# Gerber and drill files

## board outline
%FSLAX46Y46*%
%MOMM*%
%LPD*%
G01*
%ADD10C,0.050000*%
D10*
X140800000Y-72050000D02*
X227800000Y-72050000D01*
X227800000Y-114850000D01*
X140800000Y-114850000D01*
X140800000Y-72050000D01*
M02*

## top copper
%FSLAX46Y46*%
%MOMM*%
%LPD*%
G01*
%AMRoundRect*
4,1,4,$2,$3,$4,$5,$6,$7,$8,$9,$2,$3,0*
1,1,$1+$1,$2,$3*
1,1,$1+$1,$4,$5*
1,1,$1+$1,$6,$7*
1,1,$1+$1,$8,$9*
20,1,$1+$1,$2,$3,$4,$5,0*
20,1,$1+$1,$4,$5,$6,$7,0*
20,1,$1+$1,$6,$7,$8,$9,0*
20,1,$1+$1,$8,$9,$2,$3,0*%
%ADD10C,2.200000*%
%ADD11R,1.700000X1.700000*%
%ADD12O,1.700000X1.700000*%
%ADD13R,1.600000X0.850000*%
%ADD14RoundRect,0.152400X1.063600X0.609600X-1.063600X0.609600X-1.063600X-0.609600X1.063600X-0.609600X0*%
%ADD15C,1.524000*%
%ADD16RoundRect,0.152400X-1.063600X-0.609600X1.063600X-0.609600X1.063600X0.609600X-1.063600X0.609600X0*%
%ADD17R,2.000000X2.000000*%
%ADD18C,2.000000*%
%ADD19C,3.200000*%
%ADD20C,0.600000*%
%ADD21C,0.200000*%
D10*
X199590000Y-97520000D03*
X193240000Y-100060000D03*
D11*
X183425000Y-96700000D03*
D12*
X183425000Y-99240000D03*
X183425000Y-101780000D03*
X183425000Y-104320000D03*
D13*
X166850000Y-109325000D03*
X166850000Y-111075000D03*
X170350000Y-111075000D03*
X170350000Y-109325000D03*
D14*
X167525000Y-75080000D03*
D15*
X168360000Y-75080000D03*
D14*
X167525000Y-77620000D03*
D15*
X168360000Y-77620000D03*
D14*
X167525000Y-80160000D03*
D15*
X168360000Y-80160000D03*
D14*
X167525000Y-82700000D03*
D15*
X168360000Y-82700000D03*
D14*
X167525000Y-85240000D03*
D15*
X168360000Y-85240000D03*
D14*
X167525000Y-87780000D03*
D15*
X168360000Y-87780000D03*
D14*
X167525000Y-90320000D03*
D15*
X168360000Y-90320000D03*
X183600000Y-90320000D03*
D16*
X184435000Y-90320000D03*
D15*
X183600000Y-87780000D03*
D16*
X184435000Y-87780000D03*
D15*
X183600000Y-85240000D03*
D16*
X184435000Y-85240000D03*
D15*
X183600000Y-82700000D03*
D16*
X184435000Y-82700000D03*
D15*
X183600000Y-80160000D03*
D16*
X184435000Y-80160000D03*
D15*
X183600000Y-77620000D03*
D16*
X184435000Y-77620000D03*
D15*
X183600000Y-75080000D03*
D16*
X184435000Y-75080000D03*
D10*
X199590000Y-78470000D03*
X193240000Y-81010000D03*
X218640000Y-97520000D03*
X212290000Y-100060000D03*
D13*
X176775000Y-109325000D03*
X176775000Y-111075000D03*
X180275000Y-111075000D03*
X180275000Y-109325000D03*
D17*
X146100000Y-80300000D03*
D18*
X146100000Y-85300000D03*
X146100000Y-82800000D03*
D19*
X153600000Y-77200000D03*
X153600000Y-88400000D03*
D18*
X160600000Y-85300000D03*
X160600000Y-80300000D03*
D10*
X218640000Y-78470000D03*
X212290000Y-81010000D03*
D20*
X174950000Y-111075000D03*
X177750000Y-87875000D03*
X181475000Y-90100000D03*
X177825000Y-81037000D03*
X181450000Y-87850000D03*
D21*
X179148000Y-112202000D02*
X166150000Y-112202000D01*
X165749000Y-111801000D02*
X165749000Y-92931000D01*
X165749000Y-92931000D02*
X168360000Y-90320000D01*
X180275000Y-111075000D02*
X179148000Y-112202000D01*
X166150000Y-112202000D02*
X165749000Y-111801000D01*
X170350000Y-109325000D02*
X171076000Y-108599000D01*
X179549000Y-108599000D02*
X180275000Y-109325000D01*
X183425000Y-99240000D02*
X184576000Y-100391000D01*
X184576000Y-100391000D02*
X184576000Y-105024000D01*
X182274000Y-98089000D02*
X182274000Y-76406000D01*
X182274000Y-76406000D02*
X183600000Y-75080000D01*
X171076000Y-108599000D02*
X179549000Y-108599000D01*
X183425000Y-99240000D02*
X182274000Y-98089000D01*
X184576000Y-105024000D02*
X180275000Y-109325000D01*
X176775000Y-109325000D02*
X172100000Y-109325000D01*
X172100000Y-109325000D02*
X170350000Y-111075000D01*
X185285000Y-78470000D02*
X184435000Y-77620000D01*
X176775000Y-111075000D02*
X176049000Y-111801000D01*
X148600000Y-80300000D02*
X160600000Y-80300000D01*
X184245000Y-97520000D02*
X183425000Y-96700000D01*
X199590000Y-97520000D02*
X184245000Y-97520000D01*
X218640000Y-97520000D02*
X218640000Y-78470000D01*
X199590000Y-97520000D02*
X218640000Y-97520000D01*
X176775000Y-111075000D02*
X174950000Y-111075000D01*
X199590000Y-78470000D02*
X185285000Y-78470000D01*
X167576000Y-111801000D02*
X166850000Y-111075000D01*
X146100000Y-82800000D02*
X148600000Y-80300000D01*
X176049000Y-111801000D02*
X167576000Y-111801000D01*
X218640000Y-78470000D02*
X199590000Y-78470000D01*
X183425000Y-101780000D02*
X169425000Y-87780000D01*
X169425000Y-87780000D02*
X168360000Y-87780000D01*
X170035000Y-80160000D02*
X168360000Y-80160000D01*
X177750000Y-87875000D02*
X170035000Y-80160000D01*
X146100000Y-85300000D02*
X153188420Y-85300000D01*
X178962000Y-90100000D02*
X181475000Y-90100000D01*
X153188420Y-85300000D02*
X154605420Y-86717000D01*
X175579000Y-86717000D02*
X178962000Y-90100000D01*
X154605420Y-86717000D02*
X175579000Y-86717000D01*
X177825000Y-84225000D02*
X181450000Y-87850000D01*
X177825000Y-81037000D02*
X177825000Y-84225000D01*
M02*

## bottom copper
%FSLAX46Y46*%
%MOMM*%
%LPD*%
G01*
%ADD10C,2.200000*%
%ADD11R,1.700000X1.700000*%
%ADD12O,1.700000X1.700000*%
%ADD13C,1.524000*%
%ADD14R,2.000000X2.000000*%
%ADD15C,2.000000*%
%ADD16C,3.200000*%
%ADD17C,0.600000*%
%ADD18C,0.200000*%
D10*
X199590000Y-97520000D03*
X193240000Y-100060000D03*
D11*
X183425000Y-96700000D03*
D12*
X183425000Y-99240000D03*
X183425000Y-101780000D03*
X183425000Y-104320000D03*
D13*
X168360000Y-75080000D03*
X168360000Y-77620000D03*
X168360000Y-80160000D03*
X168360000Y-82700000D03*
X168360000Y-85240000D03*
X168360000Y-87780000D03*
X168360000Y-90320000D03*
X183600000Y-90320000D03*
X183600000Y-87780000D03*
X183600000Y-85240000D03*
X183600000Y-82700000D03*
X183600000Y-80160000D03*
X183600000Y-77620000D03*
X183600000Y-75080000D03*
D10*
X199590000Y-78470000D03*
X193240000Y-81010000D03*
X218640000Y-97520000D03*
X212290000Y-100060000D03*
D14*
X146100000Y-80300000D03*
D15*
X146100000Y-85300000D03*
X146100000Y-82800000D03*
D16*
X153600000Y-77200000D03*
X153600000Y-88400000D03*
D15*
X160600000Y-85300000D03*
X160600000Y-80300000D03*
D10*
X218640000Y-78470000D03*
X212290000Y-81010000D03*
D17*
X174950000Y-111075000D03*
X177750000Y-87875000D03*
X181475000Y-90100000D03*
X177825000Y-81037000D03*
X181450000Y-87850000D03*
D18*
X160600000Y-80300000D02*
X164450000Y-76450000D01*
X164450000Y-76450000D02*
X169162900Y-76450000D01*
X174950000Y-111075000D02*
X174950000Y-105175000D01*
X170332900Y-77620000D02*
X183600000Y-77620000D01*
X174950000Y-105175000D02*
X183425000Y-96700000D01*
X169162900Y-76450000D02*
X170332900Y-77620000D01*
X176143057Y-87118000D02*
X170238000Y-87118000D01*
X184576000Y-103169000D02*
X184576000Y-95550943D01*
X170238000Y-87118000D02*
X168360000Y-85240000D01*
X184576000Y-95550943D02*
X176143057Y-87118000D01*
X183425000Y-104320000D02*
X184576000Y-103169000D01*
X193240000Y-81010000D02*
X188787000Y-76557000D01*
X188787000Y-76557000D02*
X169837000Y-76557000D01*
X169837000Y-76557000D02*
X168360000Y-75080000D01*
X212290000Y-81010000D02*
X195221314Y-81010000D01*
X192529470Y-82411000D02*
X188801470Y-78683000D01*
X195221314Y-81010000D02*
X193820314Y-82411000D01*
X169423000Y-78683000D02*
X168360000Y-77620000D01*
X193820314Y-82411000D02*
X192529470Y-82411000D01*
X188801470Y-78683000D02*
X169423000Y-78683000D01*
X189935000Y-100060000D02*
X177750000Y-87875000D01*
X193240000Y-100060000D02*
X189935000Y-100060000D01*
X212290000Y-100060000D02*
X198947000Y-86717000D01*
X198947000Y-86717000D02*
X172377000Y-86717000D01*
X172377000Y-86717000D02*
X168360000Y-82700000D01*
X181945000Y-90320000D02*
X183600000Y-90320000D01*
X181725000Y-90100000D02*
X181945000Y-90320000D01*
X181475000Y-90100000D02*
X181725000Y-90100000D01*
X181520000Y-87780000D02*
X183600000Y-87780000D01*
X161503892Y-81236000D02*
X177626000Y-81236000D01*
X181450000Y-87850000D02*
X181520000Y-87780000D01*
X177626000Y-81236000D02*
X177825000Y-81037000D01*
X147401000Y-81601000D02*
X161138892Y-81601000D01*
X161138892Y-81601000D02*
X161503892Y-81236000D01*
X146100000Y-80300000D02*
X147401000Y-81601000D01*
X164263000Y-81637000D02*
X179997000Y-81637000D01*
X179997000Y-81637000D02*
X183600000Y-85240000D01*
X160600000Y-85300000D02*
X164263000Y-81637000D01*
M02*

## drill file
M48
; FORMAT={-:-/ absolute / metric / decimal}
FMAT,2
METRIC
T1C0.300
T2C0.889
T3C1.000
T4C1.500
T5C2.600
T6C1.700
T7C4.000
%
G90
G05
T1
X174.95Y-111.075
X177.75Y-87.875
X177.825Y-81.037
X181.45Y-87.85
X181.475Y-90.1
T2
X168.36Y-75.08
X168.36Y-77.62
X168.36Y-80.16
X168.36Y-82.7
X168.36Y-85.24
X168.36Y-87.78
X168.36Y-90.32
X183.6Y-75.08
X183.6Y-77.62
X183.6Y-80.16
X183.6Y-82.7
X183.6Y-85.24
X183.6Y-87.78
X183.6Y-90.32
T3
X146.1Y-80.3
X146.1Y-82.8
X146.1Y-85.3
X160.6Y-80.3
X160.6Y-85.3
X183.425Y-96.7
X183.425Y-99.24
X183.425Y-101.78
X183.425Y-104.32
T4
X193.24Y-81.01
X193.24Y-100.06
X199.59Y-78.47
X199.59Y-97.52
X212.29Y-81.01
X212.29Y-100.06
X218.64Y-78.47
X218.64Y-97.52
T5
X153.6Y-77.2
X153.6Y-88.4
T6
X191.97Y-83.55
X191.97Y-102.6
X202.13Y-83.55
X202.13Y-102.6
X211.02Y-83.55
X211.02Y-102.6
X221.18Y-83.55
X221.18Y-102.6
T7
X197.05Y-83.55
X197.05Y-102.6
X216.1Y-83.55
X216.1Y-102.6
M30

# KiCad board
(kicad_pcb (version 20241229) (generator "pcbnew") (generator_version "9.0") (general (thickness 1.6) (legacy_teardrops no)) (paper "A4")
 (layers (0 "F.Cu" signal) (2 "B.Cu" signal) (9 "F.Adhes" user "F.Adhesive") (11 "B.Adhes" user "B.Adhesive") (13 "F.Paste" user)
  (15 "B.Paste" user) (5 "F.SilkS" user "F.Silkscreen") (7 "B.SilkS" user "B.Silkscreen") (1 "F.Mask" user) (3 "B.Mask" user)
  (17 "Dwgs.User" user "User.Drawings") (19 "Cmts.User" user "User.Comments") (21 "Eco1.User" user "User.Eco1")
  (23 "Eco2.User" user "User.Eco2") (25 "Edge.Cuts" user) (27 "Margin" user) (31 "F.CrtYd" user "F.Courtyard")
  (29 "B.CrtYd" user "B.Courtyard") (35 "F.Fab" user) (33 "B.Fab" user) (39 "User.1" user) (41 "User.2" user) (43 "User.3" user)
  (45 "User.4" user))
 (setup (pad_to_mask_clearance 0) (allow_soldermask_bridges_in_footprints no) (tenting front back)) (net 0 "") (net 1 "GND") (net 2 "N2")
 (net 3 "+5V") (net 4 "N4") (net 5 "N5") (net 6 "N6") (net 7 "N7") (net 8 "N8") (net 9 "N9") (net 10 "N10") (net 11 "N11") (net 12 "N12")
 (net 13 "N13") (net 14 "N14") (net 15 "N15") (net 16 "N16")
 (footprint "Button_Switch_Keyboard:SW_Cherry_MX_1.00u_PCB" (layer "F.Cu") (at 199.59 97.52)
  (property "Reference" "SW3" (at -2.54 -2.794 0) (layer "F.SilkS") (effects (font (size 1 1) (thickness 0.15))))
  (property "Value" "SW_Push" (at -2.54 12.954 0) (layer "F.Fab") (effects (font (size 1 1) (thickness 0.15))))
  (pad "" np_thru_hole circle (at -7.62 5.08) (size 1.7 1.7) (drill 1.7) (layers "*.Cu" "*.Mask"))
  (pad "" np_thru_hole circle (at -2.54 5.08) (size 4 4) (drill 4) (layers "*.Cu" "*.Mask"))
  (pad "" np_thru_hole circle (at 2.54 5.08) (size 1.7 1.7) (drill 1.7) (layers "*.Cu" "*.Mask"))
  (pad "1" thru_hole circle (at 0 0) (size 2.2 2.2) (drill 1.5) (layers "*.Cu" "*.Mask") (remove_unused_layers no) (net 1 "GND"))
  (pad "2" thru_hole circle (at -6.35 2.54) (size 2.2 2.2) (drill 1.5) (layers "*.Cu" "*.Mask") (remove_unused_layers no) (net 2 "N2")))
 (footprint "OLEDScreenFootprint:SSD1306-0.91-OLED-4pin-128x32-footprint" (layer "F.Cu") (at 146.925 94.51)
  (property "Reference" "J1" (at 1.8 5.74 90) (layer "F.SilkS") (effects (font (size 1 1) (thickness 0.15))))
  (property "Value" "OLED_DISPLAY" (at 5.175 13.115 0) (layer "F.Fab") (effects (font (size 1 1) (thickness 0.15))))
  (pad "1" thru_hole rect (at 36.5 2.19) (size 1.7 1.7) (drill 1) (layers "*.Cu" "*.Mask") (remove_unused_layers no) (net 1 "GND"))
  (pad "2" thru_hole oval (at 36.5 4.73) (size 1.7 1.7) (drill 1) (layers "*.Cu" "*.Mask") (remove_unused_layers no) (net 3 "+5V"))
  (pad "3" thru_hole oval (at 36.5 7.27) (size 1.7 1.7) (drill 1) (layers "*.Cu" "*.Mask") (remove_unused_layers no) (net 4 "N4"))
  (pad "4" thru_hole oval (at 36.5 9.81) (size 1.7 1.7) (drill 1) (layers "*.Cu" "*.Mask") (remove_unused_layers no) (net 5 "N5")))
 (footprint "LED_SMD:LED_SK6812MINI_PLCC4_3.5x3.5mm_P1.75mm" (layer "F.Cu") (at 168.6 110.2)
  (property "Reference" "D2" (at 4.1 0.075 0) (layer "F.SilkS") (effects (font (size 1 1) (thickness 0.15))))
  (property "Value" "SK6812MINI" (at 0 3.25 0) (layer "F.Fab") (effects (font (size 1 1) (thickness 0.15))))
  (pad "1" smd rect (at -1.75 -0.875) (size 1.6 0.85) (layers "F.Cu" "F.Mask" "F.Paste") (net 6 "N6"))
  (pad "2" smd rect (at -1.75 0.875) (size 1.6 0.85) (layers "F.Cu" "F.Mask" "F.Paste") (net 1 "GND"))
  (pad "3" smd rect (at 1.75 0.875) (size 1.6 0.85) (layers "F.Cu" "F.Mask" "F.Paste") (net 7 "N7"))
  (pad "4" smd rect (at 1.75 -0.875) (size 1.6 0.85) (layers "F.Cu" "F.Mask" "F.Paste") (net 3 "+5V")))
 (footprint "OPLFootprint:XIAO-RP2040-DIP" (layer "F.Cu") (at 175.98 82.7)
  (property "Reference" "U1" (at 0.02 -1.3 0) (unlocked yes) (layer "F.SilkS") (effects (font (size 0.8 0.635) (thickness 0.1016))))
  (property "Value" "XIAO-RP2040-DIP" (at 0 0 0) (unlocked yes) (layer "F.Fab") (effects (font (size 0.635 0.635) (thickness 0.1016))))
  (pad "1" smd roundrect (at -8.455 -7.62 180) (size 2.432 1.524) (layers "F.Cu" "F.Mask") (roundrect_rratio 0.1) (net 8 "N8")
   (thermal_bridge_angle 45))
  (pad "1" thru_hole circle (at -7.62 -7.62 180) (size 1.524 1.524) (drill 0.889) (layers "*.Cu" "*.Mask") (remove_unused_layers no)
   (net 8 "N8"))
  (pad "2" smd roundrect (at -8.455 -5.08 180) (size 2.432 1.524) (layers "F.Cu" "F.Mask") (roundrect_rratio 0.1) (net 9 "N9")
   (thermal_bridge_angle 45))
  (pad "2" thru_hole circle (at -7.62 -5.08 180) (size 1.524 1.524) (drill 0.889) (layers "*.Cu" "*.Mask") (remove_unused_layers no)
   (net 9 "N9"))
  (pad "3" smd roundrect (at -8.455 -2.54 180) (size 2.432 1.524) (layers "F.Cu" "F.Mask") (roundrect_rratio 0.1) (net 2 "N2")
   (thermal_bridge_angle 45))
  (pad "3" thru_hole circle (at -7.62 -2.54 180) (size 1.524 1.524) (drill 0.889) (layers "*.Cu" "*.Mask") (remove_unused_layers no)
   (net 2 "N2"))
  (pad "4" smd roundrect (at -8.455 0 180) (size 2.432 1.524) (layers "F.Cu" "F.Mask") (roundrect_rratio 0.1) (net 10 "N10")
   (thermal_bridge_angle 45))
  (pad "4" thru_hole circle (at -7.62 0 180) (size 1.524 1.524) (drill 0.889) (layers "*.Cu" "*.Mask") (remove_unused_layers no)
   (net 10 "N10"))
  (pad "5" smd roundrect (at -8.455 2.54 180) (size 2.432 1.524) (layers "F.Cu" "F.Mask") (roundrect_rratio 0.1) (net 5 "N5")
   (thermal_bridge_angle 45))
  (pad "5" thru_hole circle (at -7.62 2.54 180) (size 1.524 1.524) (drill 0.889) (layers "*.Cu" "*.Mask") (remove_unused_layers no)
   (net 5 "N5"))
  (pad "6" smd roundrect (at -8.455 5.08 180) (size 2.432 1.524) (layers "F.Cu" "F.Mask") (roundrect_rratio 0.1) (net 4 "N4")
   (thermal_bridge_angle 45))
  (pad "6" thru_hole circle (at -7.62 5.08 180) (size 1.524 1.524) (drill 0.889) (layers "*.Cu" "*.Mask") (remove_unused_layers no)
   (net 4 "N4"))
  (pad "7" smd roundrect (at -8.455 7.62 180) (size 2.432 1.524) (layers "F.Cu" "F.Mask") (roundrect_rratio 0.1) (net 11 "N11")
   (thermal_bridge_angle 45))
  (pad "7" thru_hole circle (at -7.62 7.62 180) (size 1.524 1.524) (drill 0.889) (layers "*.Cu" "*.Mask") (remove_unused_layers no)
   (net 11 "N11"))
  (pad "8" thru_hole circle (at 7.62 7.62) (size 1.524 1.524) (drill 0.889) (layers "*.Cu" "*.Mask") (remove_unused_layers no)
   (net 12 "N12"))
  (pad "8" smd roundrect (at 8.455 7.62) (size 2.432 1.524) (layers "F.Cu" "F.Mask") (roundrect_rratio 0.1) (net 12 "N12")
   (thermal_bridge_angle 45))
  (pad "9" thru_hole circle (at 7.62 5.08) (size 1.524 1.524) (drill 0.889) (layers "*.Cu" "*.Mask") (remove_unused_layers no)
   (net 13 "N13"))
  (pad "9" smd roundrect (at 8.455 5.08) (size 2.432 1.524) (layers "F.Cu" "F.Mask") (roundrect_rratio 0.1) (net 13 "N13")
   (thermal_bridge_angle 45))
  (pad "10" thru_hole circle (at 7.62 2.54) (size 1.524 1.524) (drill 0.889) (layers "*.Cu" "*.Mask") (remove_unused_layers no)
   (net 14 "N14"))
  (pad "10" smd roundrect (at 8.455 2.54) (size 2.432 1.524) (layers "F.Cu" "F.Mask") (roundrect_rratio 0.1) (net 14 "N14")
   (thermal_bridge_angle 45))
  (pad "11" thru_hole circle (at 7.62 0) (size 1.524 1.524) (drill 0.889) (layers "*.Cu" "*.Mask") (remove_unused_layers no) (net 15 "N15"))
  (pad "11" smd roundrect (at 8.455 0) (size 2.432 1.524) (layers "F.Cu" "F.Mask") (roundrect_rratio 0.1) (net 15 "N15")
   (thermal_bridge_angle 45))
  (pad "12" thru_hole circle (at 7.62 -2.54) (size 1.524 1.524) (drill 0.889) (layers "*.Cu" "*.Mask") (remove_unused_layers no)
   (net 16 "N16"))
  (pad "12" smd roundrect (at 8.455 -2.54) (size 2.432 1.524) (layers "F.Cu" "F.Mask") (roundrect_rratio 0.1) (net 16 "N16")
   (thermal_bridge_angle 45))
  (pad "13" thru_hole circle (at 7.62 -5.08) (size 1.524 1.524) (drill 0.889) (layers "*.Cu" "*.Mask") (remove_unused_layers no)
   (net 1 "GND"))
  (pad "13" smd roundrect (at 8.455 -5.08) (size 2.432 1.524) (layers "F.Cu" "F.Mask") (roundrect_rratio 0.1) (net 1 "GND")
   (thermal_bridge_angle 45))
  (pad "14" thru_hole circle (at 7.62 -7.62) (size 1.524 1.524) (drill 0.889) (layers "*.Cu" "*.Mask") (remove_unused_layers no)
   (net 3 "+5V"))
  (pad "14" smd roundrect (at 8.455 -7.62) (size 2.432 1.524) (layers "F.Cu" "F.Mask") (roundrect_rratio 0.1) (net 3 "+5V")
   (thermal_bridge_angle 45)))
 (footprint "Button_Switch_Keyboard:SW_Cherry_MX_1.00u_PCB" (layer "F.Cu") (at 199.59 78.47)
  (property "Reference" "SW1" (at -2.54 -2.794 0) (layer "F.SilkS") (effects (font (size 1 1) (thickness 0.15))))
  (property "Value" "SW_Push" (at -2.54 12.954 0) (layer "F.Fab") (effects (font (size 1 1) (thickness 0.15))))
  (pad "" np_thru_hole circle (at -7.62 5.08) (size 1.7 1.7) (drill 1.7) (layers "*.Cu" "*.Mask"))
  (pad "" np_thru_hole circle (at -2.54 5.08) (size 4 4) (drill 4) (layers "*.Cu" "*.Mask"))
  (pad "" np_thru_hole circle (at 2.54 5.08) (size 1.7 1.7) (drill 1.7) (layers "*.Cu" "*.Mask"))
  (pad "1" thru_hole circle (at 0 0) (size 2.2 2.2) (drill 1.5) (layers "*.Cu" "*.Mask") (remove_unused_layers no) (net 1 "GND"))
  (pad "2" thru_hole circle (at -6.35 2.54) (size 2.2 2.2) (drill 1.5) (layers "*.Cu" "*.Mask") (remove_unused_layers no) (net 8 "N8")))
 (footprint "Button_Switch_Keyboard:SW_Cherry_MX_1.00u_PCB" (layer "F.Cu") (at 218.64 97.52)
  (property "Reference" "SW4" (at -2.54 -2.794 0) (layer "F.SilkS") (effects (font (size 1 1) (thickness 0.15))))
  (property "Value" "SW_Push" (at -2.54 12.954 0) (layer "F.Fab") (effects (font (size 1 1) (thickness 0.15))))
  (pad "" np_thru_hole circle (at -7.62 5.08) (size 1.7 1.7) (drill 1.7) (layers "*.Cu" "*.Mask"))
  (pad "" np_thru_hole circle (at -2.54 5.08) (size 4 4) (drill 4) (layers "*.Cu" "*.Mask"))
  (pad "" np_thru_hole circle (at 2.54 5.08) (size 1.7 1.7) (drill 1.7) (layers "*.Cu" "*.Mask"))
  (pad "1" thru_hole circle (at 0 0) (size 2.2 2.2) (drill 1.5) (layers "*.Cu" "*.Mask") (remove_unused_layers no) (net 1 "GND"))
  (pad "2" thru_hole circle (at -6.35 2.54) (size 2.2 2.2) (drill 1.5) (layers "*.Cu" "*.Mask") (remove_unused_layers no) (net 10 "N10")))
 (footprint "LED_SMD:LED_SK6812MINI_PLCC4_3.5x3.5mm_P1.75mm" (layer "F.Cu") (at 178.525 110.2)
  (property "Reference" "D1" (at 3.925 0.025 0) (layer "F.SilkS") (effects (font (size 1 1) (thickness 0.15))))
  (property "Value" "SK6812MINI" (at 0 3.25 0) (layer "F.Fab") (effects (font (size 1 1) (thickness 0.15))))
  (pad "1" smd rect (at -1.75 -0.875) (size 1.6 0.85) (layers "F.Cu" "F.Mask" "F.Paste") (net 7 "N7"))
  (pad "2" smd rect (at -1.75 0.875) (size 1.6 0.85) (layers "F.Cu" "F.Mask" "F.Paste") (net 1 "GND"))
  (pad "3" smd rect (at 1.75 0.875) (size 1.6 0.85) (layers "F.Cu" "F.Mask" "F.Paste") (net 11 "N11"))
  (pad "4" smd rect (at 1.75 -0.875) (size 1.6 0.85) (layers "F.Cu" "F.Mask" "F.Paste") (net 3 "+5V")))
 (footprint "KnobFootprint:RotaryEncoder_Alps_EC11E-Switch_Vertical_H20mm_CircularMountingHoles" (layer "F.Cu") (at 146.1 80.3)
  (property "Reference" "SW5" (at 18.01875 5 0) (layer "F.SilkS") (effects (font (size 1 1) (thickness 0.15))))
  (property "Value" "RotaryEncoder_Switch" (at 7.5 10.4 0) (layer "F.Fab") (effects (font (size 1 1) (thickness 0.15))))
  (pad "A" thru_hole rect (at 0 0) (size 2 2) (drill 1) (layers "*.Cu" "*.Mask") (remove_unused_layers no) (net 13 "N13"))
  (pad "B" thru_hole circle (at 0 5) (size 2 2) (drill 1) (layers "*.Cu" "*.Mask") (remove_unused_layers no) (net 12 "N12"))
  (pad "C" thru_hole circle (at 0 2.5) (size 2 2) (drill 1) (layers "*.Cu" "*.Mask") (remove_unused_layers no) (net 1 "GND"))
  (pad "MP" thru_hole circle (at 7.5 -3.1) (size 3.2 3.2) (drill 2.6) (layers "*.Cu" "*.Mask") (remove_unused_layers no))
  (pad "MP" thru_hole circle (at 7.5 8.1) (size 3.2 3.2) (drill 2.6) (layers "*.Cu" "*.Mask") (remove_unused_layers no))
  (pad "S1" thru_hole circle (at 14.5 5) (size 2 2) (drill 1) (layers "*.Cu" "*.Mask") (remove_unused_layers no) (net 14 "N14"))
  (pad "S2" thru_hole circle (at 14.5 0) (size 2 2) (drill 1) (layers "*.Cu" "*.Mask") (remove_unused_layers no) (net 1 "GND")))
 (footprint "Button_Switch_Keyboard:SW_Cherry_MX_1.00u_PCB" (layer "F.Cu") (at 218.64 78.47)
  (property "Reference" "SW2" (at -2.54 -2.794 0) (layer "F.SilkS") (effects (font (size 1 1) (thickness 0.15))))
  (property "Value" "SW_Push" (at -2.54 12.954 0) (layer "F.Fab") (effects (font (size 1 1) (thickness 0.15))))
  (pad "" np_thru_hole circle (at -7.62 5.08) (size 1.7 1.7) (drill 1.7) (layers "*.Cu" "*.Mask"))
  (pad "" np_thru_hole circle (at -2.54 5.08) (size 4 4) (drill 4) (layers "*.Cu" "*.Mask"))
  (pad "" np_thru_hole circle (at 2.54 5.08) (size 1.7 1.7) (drill 1.7) (layers "*.Cu" "*.Mask"))
  (pad "1" thru_hole circle (at 0 0) (size 2.2 2.2) (drill 1.5) (layers "*.Cu" "*.Mask") (remove_unused_layers no) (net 1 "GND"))
  (pad "2" thru_hole circle (at -6.35 2.54) (size 2.2 2.2) (drill 1.5) (layers "*.Cu" "*.Mask") (remove_unused_layers no) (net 9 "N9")))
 (gr_rect (start 140.8 72.05) (end 227.8 114.85) (stroke (width 0.05) (type default)) (fill no) (layer "Edge.Cuts"))
 (segment (start 179.148 112.202) (end 166.15 112.202) (width 0.2) (layer "F.Cu") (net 11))
 (segment (start 165.749 111.801) (end 165.749 92.931) (width 0.2) (layer "F.Cu") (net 11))
 (segment (start 165.749 92.931) (end 168.36 90.32) (width 0.2) (layer "F.Cu") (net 11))
 (segment (start 180.275 111.075) (end 179.148 112.202) (width 0.2) (layer "F.Cu") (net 11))
 (segment (start 166.15 112.202) (end 165.749 111.801) (width 0.2) (layer "F.Cu") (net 11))
 (segment (start 170.35 109.325) (end 171.076 108.599) (width 0.2) (layer "F.Cu") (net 3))
 (segment (start 179.549 108.599) (end 180.275 109.325) (width 0.2) (layer "F.Cu") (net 3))
 (segment (start 183.425 99.24) (end 184.576 100.391) (width 0.2) (layer "F.Cu") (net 3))
 (segment (start 184.576 100.391) (end 184.576 105.024) (width 0.2) (layer "F.Cu") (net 3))
 (segment (start 182.274 98.089) (end 182.274 76.406) (width 0.2) (layer "F.Cu") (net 3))
 (segment (start 182.274 76.406) (end 183.6 75.08) (width 0.2) (layer "F.Cu") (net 3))
 (segment (start 171.076 108.599) (end 179.549 108.599) (width 0.2) (layer "F.Cu") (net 3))
 (segment (start 183.425 99.24) (end 182.274 98.089) (width 0.2) (layer "F.Cu") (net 3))
 (segment (start 184.576 105.024) (end 180.275 109.325) (width 0.2) (layer "F.Cu") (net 3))
 (segment (start 176.775 109.325) (end 172.1 109.325) (width 0.2) (layer "F.Cu") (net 7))
 (segment (start 172.1 109.325) (end 170.35 111.075) (width 0.2) (layer "F.Cu") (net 7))
 (segment (start 185.285 78.47) (end 184.435 77.62) (width 0.2) (layer "F.Cu") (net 1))
 (segment (start 176.775 111.075) (end 176.049 111.801) (width 0.2) (layer "F.Cu") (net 1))
 (segment (start 148.6 80.3) (end 160.6 80.3) (width 0.2) (layer "F.Cu") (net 1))
 (segment (start 184.245 97.52) (end 183.425 96.7) (width 0.2) (layer "F.Cu") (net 1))
 (segment (start 199.59 97.52) (end 184.245 97.52) (width 0.2) (layer "F.Cu") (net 1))
 (segment (start 218.64 97.52) (end 218.64 78.47) (width 0.2) (layer "F.Cu") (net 1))
 (segment (start 199.59 97.52) (end 218.64 97.52) (width 0.2) (layer "F.Cu") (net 1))
 (segment (start 176.775 111.075) (end 174.95 111.075) (width 0.2) (layer "F.Cu") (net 1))
 (segment (start 199.59 78.47) (end 185.285 78.47) (width 0.2) (layer "F.Cu") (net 1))
 (segment (start 167.576 111.801) (end 166.85 111.075) (width 0.2) (layer "F.Cu") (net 1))
 (segment (start 146.1 82.8) (end 148.6 80.3) (width 0.2) (layer "F.Cu") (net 1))
 (segment (start 176.049 111.801) (end 167.576 111.801) (width 0.2) (layer "F.Cu") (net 1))
 (segment (start 218.64 78.47) (end 199.59 78.47) (width 0.2) (layer "F.Cu") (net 1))
 (via (at 174.95 111.075) (size 0.6) (drill 0.3) (layers "F.Cu" "B.Cu") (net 1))
 (segment (start 160.6 80.3) (end 164.45 76.45) (width 0.2) (layer "B.Cu") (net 1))
 (segment (start 164.45 76.45) (end 169.1629 76.45) (width 0.2) (layer "B.Cu") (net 1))
 (segment (start 174.95 111.075) (end 174.95 105.175) (width 0.2) (layer "B.Cu") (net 1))
 (segment (start 170.3329 77.62) (end 183.6 77.62) (width 0.2) (layer "B.Cu") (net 1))
 (segment (start 174.95 105.175) (end 183.425 96.7) (width 0.2) (layer "B.Cu") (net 1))
 (segment (start 169.1629 76.45) (end 170.3329 77.62) (width 0.2) (layer "B.Cu") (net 1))
 (segment (start 176.143057 87.118) (end 170.238 87.118) (width 0.2) (layer "B.Cu") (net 5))
 (segment (start 184.576 103.169) (end 184.576 95.550943) (width 0.2) (layer "B.Cu") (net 5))
 (segment (start 170.238 87.118) (end 168.36 85.24) (width 0.2) (layer "B.Cu") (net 5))
 (segment (start 184.576 95.550943) (end 176.143057 87.118) (width 0.2) (layer "B.Cu") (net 5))
 (segment (start 183.425 104.32) (end 184.576 103.169) (width 0.2) (layer "B.Cu") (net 5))
 (segment (start 183.425 101.78) (end 169.425 87.78) (width 0.2) (layer "F.Cu") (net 4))
 (segment (start 169.425 87.78) (end 168.36 87.78) (width 0.2) (layer "F.Cu") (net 4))
 (segment (start 193.24 81.01) (end 188.787 76.557) (width 0.2) (layer "B.Cu") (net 8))
 (segment (start 188.787 76.557) (end 169.837 76.557) (width 0.2) (layer "B.Cu") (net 8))
 (segment (start 169.837 76.557) (end 168.36 75.08) (width 0.2) (layer "B.Cu") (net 8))
 (segment (start 212.29 81.01) (end 195.221314 81.01) (width 0.2) (layer "B.Cu") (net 9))
 (segment (start 192.52947 82.411) (end 188.80147 78.683) (width 0.2) (layer "B.Cu") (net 9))
 (segment (start 195.221314 81.01) (end 193.820314 82.411) (width 0.2) (layer "B.Cu") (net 9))
 (segment (start 169.423 78.683) (end 168.36 77.62) (width 0.2) (layer "B.Cu") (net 9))
 (segment (start 193.820314 82.411) (end 192.52947 82.411) (width 0.2) (layer "B.Cu") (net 9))
 (segment (start 188.80147 78.683) (end 169.423 78.683) (width 0.2) (layer "B.Cu") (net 9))
 (segment (start 170.035 80.16) (end 168.36 80.16) (width 0.2) (layer "F.Cu") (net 2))
 (segment (start 177.75 87.875) (end 170.035 80.16) (width 0.2) (layer "F.Cu") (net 2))
 (via (at 177.75 87.875) (size 0.6) (drill 0.3) (layers "F.Cu" "B.Cu") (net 2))
 (segment (start 189.935 100.06) (end 177.75 87.875) (width 0.2) (layer "B.Cu") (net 2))
 (segment (start 193.24 100.06) (end 189.935 100.06) (width 0.2) (layer "B.Cu") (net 2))
 (segment (start 212.29 100.06) (end 198.947 86.717) (width 0.2) (layer "B.Cu") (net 10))
 (segment (start 198.947 86.717) (end 172.377 86.717) (width 0.2) (layer "B.Cu") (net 10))
 (segment (start 172.377 86.717) (end 168.36 82.7) (width 0.2) (layer "B.Cu") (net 10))
 (segment (start 146.1 85.3) (end 153.18842 85.3) (width 0.2) (layer "F.Cu") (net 12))
 (segment (start 178.962 90.1) (end 181.475 90.1) (width 0.2) (layer "F.Cu") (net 12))
 (segment (start 153.18842 85.3) (end 154.60542 86.717) (width 0.2) (layer "F.Cu") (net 12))
 (segment (start 175.579 86.717) (end 178.962 90.1) (width 0.2) (layer "F.Cu") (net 12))
 (segment (start 154.60542 86.717) (end 175.579 86.717) (width 0.2) (layer "F.Cu") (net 12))
 (via (at 181.475 90.1) (size 0.6) (drill 0.3) (layers "F.Cu" "B.Cu") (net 12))
 (segment (start 181.945 90.32) (end 183.6 90.32) (width 0.2) (layer "B.Cu") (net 12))
 (segment (start 181.725 90.1) (end 181.945 90.32) (width 0.2) (layer "B.Cu") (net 12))
 (segment (start 181.475 90.1) (end 181.725 90.1) (width 0.2) (layer "B.Cu") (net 12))
 (segment (start 177.825 84.225) (end 181.45 87.85) (width 0.2) (layer "F.Cu") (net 13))
 (segment (start 177.825 81.037) (end 177.825 84.225) (width 0.2) (layer "F.Cu") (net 13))
 (via (at 177.825 81.037) (size 0.6) (drill 0.3) (layers "F.Cu" "B.Cu") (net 13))
 (via (at 181.45 87.85) (size 0.6) (drill 0.3) (layers "F.Cu" "B.Cu") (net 13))
 (segment (start 181.52 87.78) (end 183.6 87.78) (width 0.2) (layer "B.Cu") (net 13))
 (segment (start 161.503892 81.236) (end 177.626 81.236) (width 0.2) (layer "B.Cu") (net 13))
 (segment (start 181.45 87.85) (end 181.52 87.78) (width 0.2) (layer "B.Cu") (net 13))
 (segment (start 177.626 81.236) (end 177.825 81.037) (width 0.2) (layer "B.Cu") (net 13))
 (segment (start 147.401 81.601) (end 161.138892 81.601) (width 0.2) (layer "B.Cu") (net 13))
 (segment (start 161.138892 81.601) (end 161.503892 81.236) (width 0.2) (layer "B.Cu") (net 13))
 (segment (start 146.1 80.3) (end 147.401 81.601) (width 0.2) (layer "B.Cu") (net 13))
 (segment (start 164.263 81.637) (end 179.997 81.637) (width 0.2) (layer "B.Cu") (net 14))
 (segment (start 179.997 81.637) (end 183.6 85.24) (width 0.2) (layer "B.Cu") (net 14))
 (segment (start 160.6 85.3) (end 164.263 81.637) (width 0.2) (layer "B.Cu") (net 14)))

